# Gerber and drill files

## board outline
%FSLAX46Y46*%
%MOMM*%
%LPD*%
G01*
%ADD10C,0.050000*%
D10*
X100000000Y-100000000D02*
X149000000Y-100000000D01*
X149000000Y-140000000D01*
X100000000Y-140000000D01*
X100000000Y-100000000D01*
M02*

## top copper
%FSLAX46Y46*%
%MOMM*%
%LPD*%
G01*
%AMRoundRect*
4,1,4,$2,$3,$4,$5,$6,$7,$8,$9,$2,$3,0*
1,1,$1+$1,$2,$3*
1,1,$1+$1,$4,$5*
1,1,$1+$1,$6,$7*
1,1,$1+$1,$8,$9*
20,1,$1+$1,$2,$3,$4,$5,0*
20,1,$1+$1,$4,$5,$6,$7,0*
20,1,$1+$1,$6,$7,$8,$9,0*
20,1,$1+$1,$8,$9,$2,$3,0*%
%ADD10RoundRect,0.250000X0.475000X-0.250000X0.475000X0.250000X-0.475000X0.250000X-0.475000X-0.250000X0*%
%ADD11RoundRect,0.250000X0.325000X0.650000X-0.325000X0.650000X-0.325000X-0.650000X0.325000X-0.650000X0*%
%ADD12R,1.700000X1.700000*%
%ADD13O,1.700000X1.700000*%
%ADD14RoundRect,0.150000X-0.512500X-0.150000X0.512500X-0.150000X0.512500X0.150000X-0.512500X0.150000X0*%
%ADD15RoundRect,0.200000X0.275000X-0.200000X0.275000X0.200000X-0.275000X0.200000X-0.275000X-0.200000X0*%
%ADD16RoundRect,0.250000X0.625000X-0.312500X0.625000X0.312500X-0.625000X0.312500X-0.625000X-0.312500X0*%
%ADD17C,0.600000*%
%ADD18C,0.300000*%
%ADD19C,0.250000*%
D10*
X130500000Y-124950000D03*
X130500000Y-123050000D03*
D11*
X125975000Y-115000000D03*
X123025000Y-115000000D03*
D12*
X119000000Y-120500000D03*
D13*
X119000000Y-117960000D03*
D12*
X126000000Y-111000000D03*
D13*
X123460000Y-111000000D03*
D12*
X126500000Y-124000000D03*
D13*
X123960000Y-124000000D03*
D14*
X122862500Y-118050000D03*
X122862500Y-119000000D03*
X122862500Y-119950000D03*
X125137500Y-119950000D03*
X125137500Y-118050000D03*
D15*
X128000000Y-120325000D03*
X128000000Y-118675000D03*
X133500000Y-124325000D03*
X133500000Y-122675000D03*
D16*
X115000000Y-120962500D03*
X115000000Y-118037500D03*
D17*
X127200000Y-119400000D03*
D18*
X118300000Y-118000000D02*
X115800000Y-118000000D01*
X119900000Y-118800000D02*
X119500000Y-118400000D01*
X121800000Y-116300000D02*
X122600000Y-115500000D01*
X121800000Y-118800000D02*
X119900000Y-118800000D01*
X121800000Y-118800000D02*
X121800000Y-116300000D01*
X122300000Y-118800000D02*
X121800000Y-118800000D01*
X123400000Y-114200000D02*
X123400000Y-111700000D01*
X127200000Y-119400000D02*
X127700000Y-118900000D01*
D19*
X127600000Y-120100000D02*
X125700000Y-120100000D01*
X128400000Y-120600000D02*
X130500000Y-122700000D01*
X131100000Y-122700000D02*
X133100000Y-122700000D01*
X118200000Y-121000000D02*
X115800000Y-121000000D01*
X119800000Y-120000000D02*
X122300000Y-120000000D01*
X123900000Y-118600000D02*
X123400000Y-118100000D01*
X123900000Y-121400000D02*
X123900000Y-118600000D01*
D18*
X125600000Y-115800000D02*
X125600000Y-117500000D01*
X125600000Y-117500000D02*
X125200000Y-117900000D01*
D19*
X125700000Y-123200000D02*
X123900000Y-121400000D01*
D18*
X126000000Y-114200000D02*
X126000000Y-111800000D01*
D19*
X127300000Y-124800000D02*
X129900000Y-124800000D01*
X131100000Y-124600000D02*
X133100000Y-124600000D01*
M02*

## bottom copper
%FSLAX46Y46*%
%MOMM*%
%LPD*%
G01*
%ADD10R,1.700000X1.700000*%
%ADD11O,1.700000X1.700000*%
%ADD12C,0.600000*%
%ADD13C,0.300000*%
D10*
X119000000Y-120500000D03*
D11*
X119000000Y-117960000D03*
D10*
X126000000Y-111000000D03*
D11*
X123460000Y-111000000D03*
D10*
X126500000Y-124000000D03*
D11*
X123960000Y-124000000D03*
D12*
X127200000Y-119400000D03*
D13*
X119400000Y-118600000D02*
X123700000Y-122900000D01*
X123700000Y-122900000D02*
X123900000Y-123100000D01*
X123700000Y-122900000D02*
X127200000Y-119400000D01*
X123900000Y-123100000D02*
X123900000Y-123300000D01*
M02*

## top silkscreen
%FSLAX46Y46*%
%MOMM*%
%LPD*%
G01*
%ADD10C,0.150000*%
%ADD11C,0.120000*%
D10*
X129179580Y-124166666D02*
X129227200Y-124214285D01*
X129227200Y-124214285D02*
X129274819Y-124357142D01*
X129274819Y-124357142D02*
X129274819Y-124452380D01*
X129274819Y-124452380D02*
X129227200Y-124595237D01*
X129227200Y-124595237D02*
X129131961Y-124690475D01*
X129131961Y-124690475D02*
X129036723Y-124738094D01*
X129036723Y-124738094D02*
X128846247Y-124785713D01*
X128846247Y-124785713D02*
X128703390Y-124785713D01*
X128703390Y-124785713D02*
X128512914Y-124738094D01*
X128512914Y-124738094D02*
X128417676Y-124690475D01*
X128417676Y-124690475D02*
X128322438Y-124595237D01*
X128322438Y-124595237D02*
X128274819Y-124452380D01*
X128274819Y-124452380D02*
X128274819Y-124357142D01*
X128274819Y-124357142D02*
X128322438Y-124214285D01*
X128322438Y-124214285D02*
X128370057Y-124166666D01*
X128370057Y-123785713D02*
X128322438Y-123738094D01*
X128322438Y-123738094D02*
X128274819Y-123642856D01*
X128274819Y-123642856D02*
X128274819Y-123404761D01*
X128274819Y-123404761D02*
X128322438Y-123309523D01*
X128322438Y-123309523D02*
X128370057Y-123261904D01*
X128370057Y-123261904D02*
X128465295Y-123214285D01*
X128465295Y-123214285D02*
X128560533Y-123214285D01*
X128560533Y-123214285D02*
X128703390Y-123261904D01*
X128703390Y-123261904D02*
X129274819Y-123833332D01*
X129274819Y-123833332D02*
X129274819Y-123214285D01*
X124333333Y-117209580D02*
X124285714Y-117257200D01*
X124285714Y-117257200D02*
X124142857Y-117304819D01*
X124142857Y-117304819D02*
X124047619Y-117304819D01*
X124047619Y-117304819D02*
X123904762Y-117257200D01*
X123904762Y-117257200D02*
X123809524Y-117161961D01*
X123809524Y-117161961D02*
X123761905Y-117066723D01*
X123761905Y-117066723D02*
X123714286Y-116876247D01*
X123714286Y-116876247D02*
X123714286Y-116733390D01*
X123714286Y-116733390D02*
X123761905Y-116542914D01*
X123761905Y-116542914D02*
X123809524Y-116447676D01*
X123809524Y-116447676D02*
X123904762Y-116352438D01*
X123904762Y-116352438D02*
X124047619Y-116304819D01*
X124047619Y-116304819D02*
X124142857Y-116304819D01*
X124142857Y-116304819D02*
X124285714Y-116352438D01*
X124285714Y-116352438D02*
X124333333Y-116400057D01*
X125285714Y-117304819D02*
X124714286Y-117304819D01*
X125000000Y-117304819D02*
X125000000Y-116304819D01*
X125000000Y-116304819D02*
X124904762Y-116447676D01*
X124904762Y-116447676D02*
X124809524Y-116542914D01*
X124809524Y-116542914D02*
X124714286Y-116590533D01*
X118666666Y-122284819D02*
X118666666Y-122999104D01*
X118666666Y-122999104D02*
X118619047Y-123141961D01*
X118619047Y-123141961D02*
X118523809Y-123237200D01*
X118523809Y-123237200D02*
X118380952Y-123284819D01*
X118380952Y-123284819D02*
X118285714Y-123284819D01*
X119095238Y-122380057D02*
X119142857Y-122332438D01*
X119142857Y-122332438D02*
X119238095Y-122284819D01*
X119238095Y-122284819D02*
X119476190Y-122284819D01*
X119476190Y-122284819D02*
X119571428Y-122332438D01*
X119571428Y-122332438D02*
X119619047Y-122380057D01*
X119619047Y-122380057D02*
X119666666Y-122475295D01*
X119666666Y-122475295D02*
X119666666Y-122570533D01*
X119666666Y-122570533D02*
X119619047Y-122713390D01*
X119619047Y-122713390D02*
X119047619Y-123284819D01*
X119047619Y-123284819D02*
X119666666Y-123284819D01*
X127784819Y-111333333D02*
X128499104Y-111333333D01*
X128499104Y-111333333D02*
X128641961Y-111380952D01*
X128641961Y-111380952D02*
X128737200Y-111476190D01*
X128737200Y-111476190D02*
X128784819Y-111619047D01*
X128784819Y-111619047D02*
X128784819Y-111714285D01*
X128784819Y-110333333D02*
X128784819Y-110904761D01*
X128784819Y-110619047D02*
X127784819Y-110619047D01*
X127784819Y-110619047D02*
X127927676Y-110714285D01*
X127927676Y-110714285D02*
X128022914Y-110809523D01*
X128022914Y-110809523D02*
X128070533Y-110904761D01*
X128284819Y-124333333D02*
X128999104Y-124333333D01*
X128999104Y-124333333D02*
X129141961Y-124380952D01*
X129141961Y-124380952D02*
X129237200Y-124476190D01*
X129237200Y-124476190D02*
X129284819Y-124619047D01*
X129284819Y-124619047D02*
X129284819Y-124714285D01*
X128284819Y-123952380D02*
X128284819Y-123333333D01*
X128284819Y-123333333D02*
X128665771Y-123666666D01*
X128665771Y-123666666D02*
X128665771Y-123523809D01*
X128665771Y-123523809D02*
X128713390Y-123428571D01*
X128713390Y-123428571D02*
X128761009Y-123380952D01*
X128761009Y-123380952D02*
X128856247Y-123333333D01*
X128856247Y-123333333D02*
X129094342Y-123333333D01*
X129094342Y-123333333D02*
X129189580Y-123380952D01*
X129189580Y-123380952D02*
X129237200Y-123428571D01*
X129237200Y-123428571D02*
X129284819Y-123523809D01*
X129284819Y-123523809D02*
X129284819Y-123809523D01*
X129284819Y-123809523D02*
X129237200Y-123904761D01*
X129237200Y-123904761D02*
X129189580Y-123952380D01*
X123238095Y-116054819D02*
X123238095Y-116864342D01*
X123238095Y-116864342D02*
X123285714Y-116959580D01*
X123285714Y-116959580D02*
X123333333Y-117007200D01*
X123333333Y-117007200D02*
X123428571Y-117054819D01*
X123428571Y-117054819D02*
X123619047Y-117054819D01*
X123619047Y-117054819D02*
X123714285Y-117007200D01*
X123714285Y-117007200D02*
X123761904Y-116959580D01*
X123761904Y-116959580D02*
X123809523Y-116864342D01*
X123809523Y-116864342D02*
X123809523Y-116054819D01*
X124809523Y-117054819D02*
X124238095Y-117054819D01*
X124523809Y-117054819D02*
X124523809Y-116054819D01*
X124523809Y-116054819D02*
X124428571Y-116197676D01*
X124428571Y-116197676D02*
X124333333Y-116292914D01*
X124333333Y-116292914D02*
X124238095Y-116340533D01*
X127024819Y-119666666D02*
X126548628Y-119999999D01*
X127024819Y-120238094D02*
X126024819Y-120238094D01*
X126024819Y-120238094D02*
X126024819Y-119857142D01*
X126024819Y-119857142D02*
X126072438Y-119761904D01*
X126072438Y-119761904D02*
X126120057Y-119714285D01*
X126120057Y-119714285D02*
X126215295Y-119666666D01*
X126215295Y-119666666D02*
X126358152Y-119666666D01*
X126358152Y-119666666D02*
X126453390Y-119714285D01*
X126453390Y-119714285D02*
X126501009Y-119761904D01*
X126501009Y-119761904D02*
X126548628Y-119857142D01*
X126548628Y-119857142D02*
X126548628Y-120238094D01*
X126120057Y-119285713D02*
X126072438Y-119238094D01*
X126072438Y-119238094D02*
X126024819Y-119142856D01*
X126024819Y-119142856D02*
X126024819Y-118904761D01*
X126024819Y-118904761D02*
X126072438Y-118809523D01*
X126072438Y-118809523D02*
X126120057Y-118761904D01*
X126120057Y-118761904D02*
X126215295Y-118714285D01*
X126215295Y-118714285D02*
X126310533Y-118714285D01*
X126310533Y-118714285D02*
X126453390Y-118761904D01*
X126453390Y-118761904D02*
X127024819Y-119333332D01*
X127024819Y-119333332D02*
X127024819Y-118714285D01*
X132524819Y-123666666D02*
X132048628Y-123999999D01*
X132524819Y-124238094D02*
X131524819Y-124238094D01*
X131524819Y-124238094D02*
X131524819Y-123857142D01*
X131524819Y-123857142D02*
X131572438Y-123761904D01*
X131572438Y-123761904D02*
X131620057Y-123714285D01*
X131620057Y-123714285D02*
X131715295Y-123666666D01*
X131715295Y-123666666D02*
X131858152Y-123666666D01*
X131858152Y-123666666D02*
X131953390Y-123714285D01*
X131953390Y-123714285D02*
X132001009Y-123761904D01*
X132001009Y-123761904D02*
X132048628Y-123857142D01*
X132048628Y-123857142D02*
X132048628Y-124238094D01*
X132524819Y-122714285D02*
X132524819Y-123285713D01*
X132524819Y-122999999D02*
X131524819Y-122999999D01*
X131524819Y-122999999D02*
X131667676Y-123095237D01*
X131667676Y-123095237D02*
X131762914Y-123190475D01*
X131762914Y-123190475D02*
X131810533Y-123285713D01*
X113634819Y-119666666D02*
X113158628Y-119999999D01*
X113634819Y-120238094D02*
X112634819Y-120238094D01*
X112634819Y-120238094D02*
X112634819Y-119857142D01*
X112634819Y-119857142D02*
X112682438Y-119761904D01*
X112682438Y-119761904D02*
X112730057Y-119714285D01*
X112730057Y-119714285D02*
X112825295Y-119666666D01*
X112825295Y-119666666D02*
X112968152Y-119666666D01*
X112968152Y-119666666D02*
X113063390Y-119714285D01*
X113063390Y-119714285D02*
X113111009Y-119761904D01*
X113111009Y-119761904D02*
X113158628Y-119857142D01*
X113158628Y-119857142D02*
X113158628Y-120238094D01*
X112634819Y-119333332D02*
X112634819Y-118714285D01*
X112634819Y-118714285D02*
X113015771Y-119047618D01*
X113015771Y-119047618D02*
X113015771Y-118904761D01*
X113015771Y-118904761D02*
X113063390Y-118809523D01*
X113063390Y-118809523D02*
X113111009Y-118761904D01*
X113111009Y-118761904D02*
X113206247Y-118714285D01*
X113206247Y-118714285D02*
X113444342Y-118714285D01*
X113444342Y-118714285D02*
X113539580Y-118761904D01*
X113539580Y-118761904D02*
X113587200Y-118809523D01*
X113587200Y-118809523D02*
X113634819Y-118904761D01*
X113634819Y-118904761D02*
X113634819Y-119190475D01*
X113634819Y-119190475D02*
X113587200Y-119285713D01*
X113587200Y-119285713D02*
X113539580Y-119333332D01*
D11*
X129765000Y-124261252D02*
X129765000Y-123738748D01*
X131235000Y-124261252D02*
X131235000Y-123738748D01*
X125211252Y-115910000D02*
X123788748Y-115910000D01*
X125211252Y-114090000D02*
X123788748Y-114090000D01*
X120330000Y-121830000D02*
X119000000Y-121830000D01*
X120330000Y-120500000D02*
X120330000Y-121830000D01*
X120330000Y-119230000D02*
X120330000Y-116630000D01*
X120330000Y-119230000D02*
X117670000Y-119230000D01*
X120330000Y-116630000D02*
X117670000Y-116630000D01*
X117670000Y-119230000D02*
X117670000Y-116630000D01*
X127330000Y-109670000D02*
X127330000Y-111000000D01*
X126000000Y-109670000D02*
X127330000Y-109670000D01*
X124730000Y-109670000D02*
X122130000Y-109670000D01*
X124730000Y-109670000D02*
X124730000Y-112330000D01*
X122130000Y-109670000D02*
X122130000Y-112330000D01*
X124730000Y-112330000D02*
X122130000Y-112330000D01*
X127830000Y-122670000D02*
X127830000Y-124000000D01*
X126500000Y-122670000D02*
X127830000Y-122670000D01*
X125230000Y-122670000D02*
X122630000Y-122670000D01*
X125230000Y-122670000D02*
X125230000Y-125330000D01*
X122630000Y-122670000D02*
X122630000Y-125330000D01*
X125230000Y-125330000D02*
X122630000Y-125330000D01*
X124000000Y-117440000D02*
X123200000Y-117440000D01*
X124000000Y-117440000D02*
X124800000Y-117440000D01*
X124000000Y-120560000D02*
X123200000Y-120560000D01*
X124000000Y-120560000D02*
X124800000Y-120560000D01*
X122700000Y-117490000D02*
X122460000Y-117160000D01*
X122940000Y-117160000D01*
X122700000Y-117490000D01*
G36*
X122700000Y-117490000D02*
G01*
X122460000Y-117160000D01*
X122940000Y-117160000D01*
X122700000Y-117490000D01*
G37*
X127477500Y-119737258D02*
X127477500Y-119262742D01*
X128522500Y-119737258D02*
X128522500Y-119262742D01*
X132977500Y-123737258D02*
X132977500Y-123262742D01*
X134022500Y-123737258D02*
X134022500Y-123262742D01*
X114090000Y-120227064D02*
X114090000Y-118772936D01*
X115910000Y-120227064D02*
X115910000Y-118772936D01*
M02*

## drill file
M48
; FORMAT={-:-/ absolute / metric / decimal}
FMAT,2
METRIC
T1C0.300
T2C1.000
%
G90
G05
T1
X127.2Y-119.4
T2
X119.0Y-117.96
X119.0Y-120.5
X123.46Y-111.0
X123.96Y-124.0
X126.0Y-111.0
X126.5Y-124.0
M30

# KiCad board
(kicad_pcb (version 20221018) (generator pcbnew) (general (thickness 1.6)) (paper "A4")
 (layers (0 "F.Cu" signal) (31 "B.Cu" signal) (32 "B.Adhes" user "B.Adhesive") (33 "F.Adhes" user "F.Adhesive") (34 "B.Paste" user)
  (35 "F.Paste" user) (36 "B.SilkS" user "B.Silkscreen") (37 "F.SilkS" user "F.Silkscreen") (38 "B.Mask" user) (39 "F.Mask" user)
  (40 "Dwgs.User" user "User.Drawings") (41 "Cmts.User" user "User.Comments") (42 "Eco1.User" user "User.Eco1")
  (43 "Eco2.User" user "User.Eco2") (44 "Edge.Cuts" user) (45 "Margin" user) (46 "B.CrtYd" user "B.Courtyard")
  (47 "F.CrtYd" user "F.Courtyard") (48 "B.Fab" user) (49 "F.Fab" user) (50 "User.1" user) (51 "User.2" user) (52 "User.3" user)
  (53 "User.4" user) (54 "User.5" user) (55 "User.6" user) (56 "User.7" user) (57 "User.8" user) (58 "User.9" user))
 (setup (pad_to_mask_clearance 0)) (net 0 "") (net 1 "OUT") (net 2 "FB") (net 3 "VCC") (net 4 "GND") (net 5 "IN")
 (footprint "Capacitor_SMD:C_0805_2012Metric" (layer "F.Cu") (at 130.5 124 90)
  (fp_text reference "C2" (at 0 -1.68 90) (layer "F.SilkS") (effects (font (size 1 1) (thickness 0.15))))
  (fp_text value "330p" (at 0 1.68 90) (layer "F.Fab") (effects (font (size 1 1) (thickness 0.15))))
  (fp_line (start -0.261252 -0.735) (end 0.261252 -0.735) (stroke (width 0.12) (type solid)) (layer "F.SilkS"))
  (fp_line (start -0.261252 0.735) (end 0.261252 0.735) (stroke (width 0.12) (type solid)) (layer "F.SilkS"))
  (pad "1" smd roundrect (at -0.95 0 90) (size 1 1.45) (layers "F.Cu" "F.Paste" "F.Mask") (roundrect_rratio 0.25) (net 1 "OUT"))
  (pad "2" smd roundrect (at 0.95 0 90) (size 1 1.45) (layers "F.Cu" "F.Paste" "F.Mask") (roundrect_rratio 0.25) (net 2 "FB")))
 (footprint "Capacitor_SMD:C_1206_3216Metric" (layer "F.Cu") (at 124.5 115 180)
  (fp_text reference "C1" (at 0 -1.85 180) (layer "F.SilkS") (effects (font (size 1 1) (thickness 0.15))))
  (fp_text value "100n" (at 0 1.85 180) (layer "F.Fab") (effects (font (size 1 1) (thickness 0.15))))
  (fp_line (start -0.711252 -0.91) (end 0.711252 -0.91) (stroke (width 0.12) (type solid)) (layer "F.SilkS"))
  (fp_line (start -0.711252 0.91) (end 0.711252 0.91) (stroke (width 0.12) (type solid)) (layer "F.SilkS"))
  (pad "1" smd roundrect (at -1.475 0 180) (size 1.15 1.8) (layers "F.Cu" "F.Paste" "F.Mask") (roundrect_rratio 0.217391) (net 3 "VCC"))
  (pad "2" smd roundrect (at 1.475 0 180) (size 1.15 1.8) (layers "F.Cu" "F.Paste" "F.Mask") (roundrect_rratio 0.217391) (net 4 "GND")))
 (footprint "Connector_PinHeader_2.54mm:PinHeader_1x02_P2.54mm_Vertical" (layer "F.Cu") (at 119 120.5 180)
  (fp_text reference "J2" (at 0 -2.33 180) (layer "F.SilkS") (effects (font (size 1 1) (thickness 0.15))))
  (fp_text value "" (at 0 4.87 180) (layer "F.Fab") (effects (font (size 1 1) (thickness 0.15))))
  (fp_line (start -1.33 -1.33) (end 0 -1.33) (stroke (width 0.12) (type solid)) (layer "F.SilkS"))
  (fp_line (start -1.33 0) (end -1.33 -1.33) (stroke (width 0.12) (type solid)) (layer "F.SilkS"))
  (fp_line (start -1.33 1.27) (end -1.33 3.87) (stroke (width 0.12) (type solid)) (layer "F.SilkS"))
  (fp_line (start -1.33 1.27) (end 1.33 1.27) (stroke (width 0.12) (type solid)) (layer "F.SilkS"))
  (fp_line (start -1.33 3.87) (end 1.33 3.87) (stroke (width 0.12) (type solid)) (layer "F.SilkS"))
  (fp_line (start 1.33 1.27) (end 1.33 3.87) (stroke (width 0.12) (type solid)) (layer "F.SilkS"))
  (pad "1" thru_hole rect (at 0 0 180) (size 1.7 1.7) (drill 1) (layers "*.Cu" "*.Mask") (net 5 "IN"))
  (pad "2" thru_hole oval (at 0 2.54 180) (size 1.7 1.7) (drill 1) (layers "*.Cu" "*.Mask") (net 4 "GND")))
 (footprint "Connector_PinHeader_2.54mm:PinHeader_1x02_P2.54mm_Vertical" (layer "F.Cu") (at 126 111 -90)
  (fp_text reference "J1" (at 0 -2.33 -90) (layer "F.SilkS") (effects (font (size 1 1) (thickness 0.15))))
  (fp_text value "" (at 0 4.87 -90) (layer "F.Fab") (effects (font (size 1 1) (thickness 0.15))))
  (fp_line (start -1.33 -1.33) (end 0 -1.33) (stroke (width 0.12) (type solid)) (layer "F.SilkS"))
  (fp_line (start -1.33 0) (end -1.33 -1.33) (stroke (width 0.12) (type solid)) (layer "F.SilkS"))
  (fp_line (start -1.33 1.27) (end -1.33 3.87) (stroke (width 0.12) (type solid)) (layer "F.SilkS"))
  (fp_line (start -1.33 1.27) (end 1.33 1.27) (stroke (width 0.12) (type solid)) (layer "F.SilkS"))
  (fp_line (start -1.33 3.87) (end 1.33 3.87) (stroke (width 0.12) (type solid)) (layer "F.SilkS"))
  (fp_line (start 1.33 1.27) (end 1.33 3.87) (stroke (width 0.12) (type solid)) (layer "F.SilkS"))
  (pad "1" thru_hole rect (at 0 0 270) (size 1.7 1.7) (drill 1) (layers "*.Cu" "*.Mask") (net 3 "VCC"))
  (pad "2" thru_hole oval (at 0 2.54 270) (size 1.7 1.7) (drill 1) (layers "*.Cu" "*.Mask") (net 4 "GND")))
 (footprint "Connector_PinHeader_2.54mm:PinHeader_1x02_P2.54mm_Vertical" (layer "F.Cu") (at 126.5 124 -90)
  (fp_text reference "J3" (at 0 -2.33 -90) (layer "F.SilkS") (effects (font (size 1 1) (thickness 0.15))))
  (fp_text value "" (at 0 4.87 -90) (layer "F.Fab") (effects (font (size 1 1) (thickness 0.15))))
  (fp_line (start -1.33 -1.33) (end 0 -1.33) (stroke (width 0.12) (type solid)) (layer "F.SilkS"))
  (fp_line (start -1.33 0) (end -1.33 -1.33) (stroke (width 0.12) (type solid)) (layer "F.SilkS"))
  (fp_line (start -1.33 1.27) (end -1.33 3.87) (stroke (width 0.12) (type solid)) (layer "F.SilkS"))
  (fp_line (start -1.33 1.27) (end 1.33 1.27) (stroke (width 0.12) (type solid)) (layer "F.SilkS"))
  (fp_line (start -1.33 3.87) (end 1.33 3.87) (stroke (width 0.12) (type solid)) (layer "F.SilkS"))
  (fp_line (start 1.33 1.27) (end 1.33 3.87) (stroke (width 0.12) (type solid)) (layer "F.SilkS"))
  (pad "1" thru_hole rect (at 0 0 270) (size 1.7 1.7) (drill 1) (layers "*.Cu" "*.Mask") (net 1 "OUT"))
  (pad "2" thru_hole oval (at 0 2.54 270) (size 1.7 1.7) (drill 1) (layers "*.Cu" "*.Mask") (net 4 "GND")))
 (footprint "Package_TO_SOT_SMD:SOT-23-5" (layer "F.Cu") (at 124 119)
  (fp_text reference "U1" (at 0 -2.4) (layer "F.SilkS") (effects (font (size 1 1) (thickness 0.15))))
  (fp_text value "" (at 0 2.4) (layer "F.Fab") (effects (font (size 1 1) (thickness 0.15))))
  (fp_line (start 0 -1.56) (end -0.8 -1.56) (stroke (width 0.12) (type solid)) (layer "F.SilkS"))
  (fp_line (start 0 -1.56) (end 0.8 -1.56) (stroke (width 0.12) (type solid)) (layer "F.SilkS"))
  (fp_line (start 0 1.56) (end -0.8 1.56) (stroke (width 0.12) (type solid)) (layer "F.SilkS"))
  (fp_line (start 0 1.56) (end 0.8 1.56) (stroke (width 0.12) (type solid)) (layer "F.SilkS"))
  (fp_poly
   (pts (xy -1.3 -1.51) (xy -1.54 -1.84) (xy -1.06 -1.84) (xy -1.3 -1.51)) (stroke (width 0.12) (type solid)) (fill solid) (layer "F.SilkS"))
  (pad "1" smd roundrect (at -1.1375 -0.95) (size 1.325 0.6) (layers "F.Cu" "F.Paste" "F.Mask") (roundrect_rratio 0.25) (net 1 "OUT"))
  (pad "2" smd roundrect (at -1.1375 0) (size 1.325 0.6) (layers "F.Cu" "F.Paste" "F.Mask") (roundrect_rratio 0.25) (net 4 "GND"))
  (pad "3" smd roundrect (at -1.1375 0.95) (size 1.325 0.6) (layers "F.Cu" "F.Paste" "F.Mask") (roundrect_rratio 0.25) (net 5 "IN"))
  (pad "4" smd roundrect (at 1.1375 0.95) (size 1.325 0.6) (layers "F.Cu" "F.Paste" "F.Mask") (roundrect_rratio 0.25) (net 2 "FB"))
  (pad "5" smd roundrect (at 1.1375 -0.95) (size 1.325 0.6) (layers "F.Cu" "F.Paste" "F.Mask") (roundrect_rratio 0.25) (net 3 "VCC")))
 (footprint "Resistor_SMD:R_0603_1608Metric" (layer "F.Cu") (at 128 119.5 90)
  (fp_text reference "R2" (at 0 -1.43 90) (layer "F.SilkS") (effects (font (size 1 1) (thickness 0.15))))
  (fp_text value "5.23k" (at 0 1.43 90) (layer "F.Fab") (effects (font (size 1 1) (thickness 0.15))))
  (fp_line (start -0.237258 -0.5225) (end 0.237258 -0.5225) (stroke (width 0.12) (type solid)) (layer "F.SilkS"))
  (fp_line (start -0.237258 0.5225) (end 0.237258 0.5225) (stroke (width 0.12) (type solid)) (layer "F.SilkS"))
  (pad "1" smd roundrect (at -0.825 0 90) (size 0.8 0.95) (layers "F.Cu" "F.Paste" "F.Mask") (roundrect_rratio 0.25) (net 2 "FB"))
  (pad "2" smd roundrect (at 0.825 0 90) (size 0.8 0.95) (layers "F.Cu" "F.Paste" "F.Mask") (roundrect_rratio 0.25) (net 4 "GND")))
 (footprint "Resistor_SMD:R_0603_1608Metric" (layer "F.Cu") (at 133.5 123.5 90)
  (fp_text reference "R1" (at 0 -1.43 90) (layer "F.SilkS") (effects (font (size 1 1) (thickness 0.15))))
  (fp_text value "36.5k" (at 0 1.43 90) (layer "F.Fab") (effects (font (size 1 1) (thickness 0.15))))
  (fp_line (start -0.237258 -0.5225) (end 0.237258 -0.5225) (stroke (width 0.12) (type solid)) (layer "F.SilkS"))
  (fp_line (start -0.237258 0.5225) (end 0.237258 0.5225) (stroke (width 0.12) (type solid)) (layer "F.SilkS"))
  (pad "1" smd roundrect (at -0.825 0 90) (size 0.8 0.95) (layers "F.Cu" "F.Paste" "F.Mask") (roundrect_rratio 0.25) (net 1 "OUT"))
  (pad "2" smd roundrect (at 0.825 0 90) (size 0.8 0.95) (layers "F.Cu" "F.Paste" "F.Mask") (roundrect_rratio 0.25) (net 2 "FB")))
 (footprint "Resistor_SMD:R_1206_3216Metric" (layer "F.Cu") (at 115 119.5 90)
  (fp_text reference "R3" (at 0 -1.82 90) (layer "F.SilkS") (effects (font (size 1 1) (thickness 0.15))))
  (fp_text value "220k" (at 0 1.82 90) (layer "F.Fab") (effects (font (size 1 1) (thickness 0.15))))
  (fp_line (start -0.727064 -0.91) (end 0.727064 -0.91) (stroke (width 0.12) (type solid)) (layer "F.SilkS"))
  (fp_line (start -0.727064 0.91) (end 0.727064 0.91) (stroke (width 0.12) (type solid)) (layer "F.SilkS"))
  (pad "1" smd roundrect (at -1.4625 0 90) (size 1.125 1.75) (layers "F.Cu" "F.Paste" "F.Mask") (roundrect_rratio 0.222222) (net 5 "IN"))
  (pad "2" smd roundrect (at 1.4625 0 90) (size 1.125 1.75) (layers "F.Cu" "F.Paste" "F.Mask") (roundrect_rratio 0.222222) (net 4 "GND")))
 (gr_rect (start 100 100) (end 149 140) (stroke (width 0.05) (type default)) (fill none) (layer "Edge.Cuts"))
 (segment (start 118.3 118) (end 115.8 118) (width 0.3) (layer "F.Cu") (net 4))
 (segment (start 119.9 118.8) (end 119.5 118.4) (width 0.3) (layer "F.Cu") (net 4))
 (segment (start 121.8 116.3) (end 122.6 115.5) (width 0.3) (layer "F.Cu") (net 4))
 (segment (start 121.8 118.8) (end 119.9 118.8) (width 0.3) (layer "F.Cu") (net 4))
 (segment (start 121.8 118.8) (end 121.8 116.3) (width 0.3) (layer "F.Cu") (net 4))
 (segment (start 122.3 118.8) (end 121.8 118.8) (width 0.3) (layer "F.Cu") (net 4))
 (segment (start 123.4 114.2) (end 123.4 111.7) (width 0.3) (layer "F.Cu") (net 4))
 (segment (start 127.2 119.4) (end 127.7 118.9) (width 0.3) (layer "F.Cu") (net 4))
 (segment (start 127.6 120.1) (end 125.7 120.1) (width 0.25) (layer "F.Cu") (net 2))
 (segment (start 128.4 120.6) (end 130.5 122.7) (width 0.25) (layer "F.Cu") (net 2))
 (segment (start 131.1 122.7) (end 133.1 122.7) (width 0.25) (layer "F.Cu") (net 2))
 (via (at 127.2 119.4) (size 0.6) (drill 0.3) (layers "F.Cu" "B.Cu") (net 4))
 (segment (start 118.2 121) (end 115.8 121) (width 0.25) (layer "F.Cu") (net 5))
 (segment (start 119.4 118.6) (end 123.7 122.9) (width 0.3) (layer "B.Cu") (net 4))
 (segment (start 119.8 120) (end 122.3 120) (width 0.25) (layer "F.Cu") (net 5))
 (segment (start 123.7 122.9) (end 123.9 123.1) (width 0.3) (layer "B.Cu") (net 4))
 (segment (start 123.7 122.9) (end 127.2 119.4) (width 0.3) (layer "B.Cu") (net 4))
 (segment (start 123.9 118.6) (end 123.4 118.1) (width 0.25) (layer "F.Cu") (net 1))
 (segment (start 123.9 121.4) (end 123.9 118.6) (width 0.25) (layer "F.Cu") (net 1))
 (segment (start 123.9 123.1) (end 123.9 123.3) (width 0.3) (layer "B.Cu") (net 4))
 (segment (start 125.6 115.8) (end 125.6 117.5) (width 0.3) (layer "F.Cu") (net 3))
 (segment (start 125.6 117.5) (end 125.2 117.9) (width 0.3) (layer "F.Cu") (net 3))
 (segment (start 125.7 123.2) (end 123.9 121.4) (width 0.25) (layer "F.Cu") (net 1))
 (segment (start 126 114.2) (end 126 111.8) (width 0.3) (layer "F.Cu") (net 3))
 (segment (start 127.3 124.8) (end 129.9 124.8) (width 0.25) (layer "F.Cu") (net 1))
 (segment (start 131.1 124.6) (end 133.1 124.6) (width 0.25) (layer "F.Cu") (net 1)))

